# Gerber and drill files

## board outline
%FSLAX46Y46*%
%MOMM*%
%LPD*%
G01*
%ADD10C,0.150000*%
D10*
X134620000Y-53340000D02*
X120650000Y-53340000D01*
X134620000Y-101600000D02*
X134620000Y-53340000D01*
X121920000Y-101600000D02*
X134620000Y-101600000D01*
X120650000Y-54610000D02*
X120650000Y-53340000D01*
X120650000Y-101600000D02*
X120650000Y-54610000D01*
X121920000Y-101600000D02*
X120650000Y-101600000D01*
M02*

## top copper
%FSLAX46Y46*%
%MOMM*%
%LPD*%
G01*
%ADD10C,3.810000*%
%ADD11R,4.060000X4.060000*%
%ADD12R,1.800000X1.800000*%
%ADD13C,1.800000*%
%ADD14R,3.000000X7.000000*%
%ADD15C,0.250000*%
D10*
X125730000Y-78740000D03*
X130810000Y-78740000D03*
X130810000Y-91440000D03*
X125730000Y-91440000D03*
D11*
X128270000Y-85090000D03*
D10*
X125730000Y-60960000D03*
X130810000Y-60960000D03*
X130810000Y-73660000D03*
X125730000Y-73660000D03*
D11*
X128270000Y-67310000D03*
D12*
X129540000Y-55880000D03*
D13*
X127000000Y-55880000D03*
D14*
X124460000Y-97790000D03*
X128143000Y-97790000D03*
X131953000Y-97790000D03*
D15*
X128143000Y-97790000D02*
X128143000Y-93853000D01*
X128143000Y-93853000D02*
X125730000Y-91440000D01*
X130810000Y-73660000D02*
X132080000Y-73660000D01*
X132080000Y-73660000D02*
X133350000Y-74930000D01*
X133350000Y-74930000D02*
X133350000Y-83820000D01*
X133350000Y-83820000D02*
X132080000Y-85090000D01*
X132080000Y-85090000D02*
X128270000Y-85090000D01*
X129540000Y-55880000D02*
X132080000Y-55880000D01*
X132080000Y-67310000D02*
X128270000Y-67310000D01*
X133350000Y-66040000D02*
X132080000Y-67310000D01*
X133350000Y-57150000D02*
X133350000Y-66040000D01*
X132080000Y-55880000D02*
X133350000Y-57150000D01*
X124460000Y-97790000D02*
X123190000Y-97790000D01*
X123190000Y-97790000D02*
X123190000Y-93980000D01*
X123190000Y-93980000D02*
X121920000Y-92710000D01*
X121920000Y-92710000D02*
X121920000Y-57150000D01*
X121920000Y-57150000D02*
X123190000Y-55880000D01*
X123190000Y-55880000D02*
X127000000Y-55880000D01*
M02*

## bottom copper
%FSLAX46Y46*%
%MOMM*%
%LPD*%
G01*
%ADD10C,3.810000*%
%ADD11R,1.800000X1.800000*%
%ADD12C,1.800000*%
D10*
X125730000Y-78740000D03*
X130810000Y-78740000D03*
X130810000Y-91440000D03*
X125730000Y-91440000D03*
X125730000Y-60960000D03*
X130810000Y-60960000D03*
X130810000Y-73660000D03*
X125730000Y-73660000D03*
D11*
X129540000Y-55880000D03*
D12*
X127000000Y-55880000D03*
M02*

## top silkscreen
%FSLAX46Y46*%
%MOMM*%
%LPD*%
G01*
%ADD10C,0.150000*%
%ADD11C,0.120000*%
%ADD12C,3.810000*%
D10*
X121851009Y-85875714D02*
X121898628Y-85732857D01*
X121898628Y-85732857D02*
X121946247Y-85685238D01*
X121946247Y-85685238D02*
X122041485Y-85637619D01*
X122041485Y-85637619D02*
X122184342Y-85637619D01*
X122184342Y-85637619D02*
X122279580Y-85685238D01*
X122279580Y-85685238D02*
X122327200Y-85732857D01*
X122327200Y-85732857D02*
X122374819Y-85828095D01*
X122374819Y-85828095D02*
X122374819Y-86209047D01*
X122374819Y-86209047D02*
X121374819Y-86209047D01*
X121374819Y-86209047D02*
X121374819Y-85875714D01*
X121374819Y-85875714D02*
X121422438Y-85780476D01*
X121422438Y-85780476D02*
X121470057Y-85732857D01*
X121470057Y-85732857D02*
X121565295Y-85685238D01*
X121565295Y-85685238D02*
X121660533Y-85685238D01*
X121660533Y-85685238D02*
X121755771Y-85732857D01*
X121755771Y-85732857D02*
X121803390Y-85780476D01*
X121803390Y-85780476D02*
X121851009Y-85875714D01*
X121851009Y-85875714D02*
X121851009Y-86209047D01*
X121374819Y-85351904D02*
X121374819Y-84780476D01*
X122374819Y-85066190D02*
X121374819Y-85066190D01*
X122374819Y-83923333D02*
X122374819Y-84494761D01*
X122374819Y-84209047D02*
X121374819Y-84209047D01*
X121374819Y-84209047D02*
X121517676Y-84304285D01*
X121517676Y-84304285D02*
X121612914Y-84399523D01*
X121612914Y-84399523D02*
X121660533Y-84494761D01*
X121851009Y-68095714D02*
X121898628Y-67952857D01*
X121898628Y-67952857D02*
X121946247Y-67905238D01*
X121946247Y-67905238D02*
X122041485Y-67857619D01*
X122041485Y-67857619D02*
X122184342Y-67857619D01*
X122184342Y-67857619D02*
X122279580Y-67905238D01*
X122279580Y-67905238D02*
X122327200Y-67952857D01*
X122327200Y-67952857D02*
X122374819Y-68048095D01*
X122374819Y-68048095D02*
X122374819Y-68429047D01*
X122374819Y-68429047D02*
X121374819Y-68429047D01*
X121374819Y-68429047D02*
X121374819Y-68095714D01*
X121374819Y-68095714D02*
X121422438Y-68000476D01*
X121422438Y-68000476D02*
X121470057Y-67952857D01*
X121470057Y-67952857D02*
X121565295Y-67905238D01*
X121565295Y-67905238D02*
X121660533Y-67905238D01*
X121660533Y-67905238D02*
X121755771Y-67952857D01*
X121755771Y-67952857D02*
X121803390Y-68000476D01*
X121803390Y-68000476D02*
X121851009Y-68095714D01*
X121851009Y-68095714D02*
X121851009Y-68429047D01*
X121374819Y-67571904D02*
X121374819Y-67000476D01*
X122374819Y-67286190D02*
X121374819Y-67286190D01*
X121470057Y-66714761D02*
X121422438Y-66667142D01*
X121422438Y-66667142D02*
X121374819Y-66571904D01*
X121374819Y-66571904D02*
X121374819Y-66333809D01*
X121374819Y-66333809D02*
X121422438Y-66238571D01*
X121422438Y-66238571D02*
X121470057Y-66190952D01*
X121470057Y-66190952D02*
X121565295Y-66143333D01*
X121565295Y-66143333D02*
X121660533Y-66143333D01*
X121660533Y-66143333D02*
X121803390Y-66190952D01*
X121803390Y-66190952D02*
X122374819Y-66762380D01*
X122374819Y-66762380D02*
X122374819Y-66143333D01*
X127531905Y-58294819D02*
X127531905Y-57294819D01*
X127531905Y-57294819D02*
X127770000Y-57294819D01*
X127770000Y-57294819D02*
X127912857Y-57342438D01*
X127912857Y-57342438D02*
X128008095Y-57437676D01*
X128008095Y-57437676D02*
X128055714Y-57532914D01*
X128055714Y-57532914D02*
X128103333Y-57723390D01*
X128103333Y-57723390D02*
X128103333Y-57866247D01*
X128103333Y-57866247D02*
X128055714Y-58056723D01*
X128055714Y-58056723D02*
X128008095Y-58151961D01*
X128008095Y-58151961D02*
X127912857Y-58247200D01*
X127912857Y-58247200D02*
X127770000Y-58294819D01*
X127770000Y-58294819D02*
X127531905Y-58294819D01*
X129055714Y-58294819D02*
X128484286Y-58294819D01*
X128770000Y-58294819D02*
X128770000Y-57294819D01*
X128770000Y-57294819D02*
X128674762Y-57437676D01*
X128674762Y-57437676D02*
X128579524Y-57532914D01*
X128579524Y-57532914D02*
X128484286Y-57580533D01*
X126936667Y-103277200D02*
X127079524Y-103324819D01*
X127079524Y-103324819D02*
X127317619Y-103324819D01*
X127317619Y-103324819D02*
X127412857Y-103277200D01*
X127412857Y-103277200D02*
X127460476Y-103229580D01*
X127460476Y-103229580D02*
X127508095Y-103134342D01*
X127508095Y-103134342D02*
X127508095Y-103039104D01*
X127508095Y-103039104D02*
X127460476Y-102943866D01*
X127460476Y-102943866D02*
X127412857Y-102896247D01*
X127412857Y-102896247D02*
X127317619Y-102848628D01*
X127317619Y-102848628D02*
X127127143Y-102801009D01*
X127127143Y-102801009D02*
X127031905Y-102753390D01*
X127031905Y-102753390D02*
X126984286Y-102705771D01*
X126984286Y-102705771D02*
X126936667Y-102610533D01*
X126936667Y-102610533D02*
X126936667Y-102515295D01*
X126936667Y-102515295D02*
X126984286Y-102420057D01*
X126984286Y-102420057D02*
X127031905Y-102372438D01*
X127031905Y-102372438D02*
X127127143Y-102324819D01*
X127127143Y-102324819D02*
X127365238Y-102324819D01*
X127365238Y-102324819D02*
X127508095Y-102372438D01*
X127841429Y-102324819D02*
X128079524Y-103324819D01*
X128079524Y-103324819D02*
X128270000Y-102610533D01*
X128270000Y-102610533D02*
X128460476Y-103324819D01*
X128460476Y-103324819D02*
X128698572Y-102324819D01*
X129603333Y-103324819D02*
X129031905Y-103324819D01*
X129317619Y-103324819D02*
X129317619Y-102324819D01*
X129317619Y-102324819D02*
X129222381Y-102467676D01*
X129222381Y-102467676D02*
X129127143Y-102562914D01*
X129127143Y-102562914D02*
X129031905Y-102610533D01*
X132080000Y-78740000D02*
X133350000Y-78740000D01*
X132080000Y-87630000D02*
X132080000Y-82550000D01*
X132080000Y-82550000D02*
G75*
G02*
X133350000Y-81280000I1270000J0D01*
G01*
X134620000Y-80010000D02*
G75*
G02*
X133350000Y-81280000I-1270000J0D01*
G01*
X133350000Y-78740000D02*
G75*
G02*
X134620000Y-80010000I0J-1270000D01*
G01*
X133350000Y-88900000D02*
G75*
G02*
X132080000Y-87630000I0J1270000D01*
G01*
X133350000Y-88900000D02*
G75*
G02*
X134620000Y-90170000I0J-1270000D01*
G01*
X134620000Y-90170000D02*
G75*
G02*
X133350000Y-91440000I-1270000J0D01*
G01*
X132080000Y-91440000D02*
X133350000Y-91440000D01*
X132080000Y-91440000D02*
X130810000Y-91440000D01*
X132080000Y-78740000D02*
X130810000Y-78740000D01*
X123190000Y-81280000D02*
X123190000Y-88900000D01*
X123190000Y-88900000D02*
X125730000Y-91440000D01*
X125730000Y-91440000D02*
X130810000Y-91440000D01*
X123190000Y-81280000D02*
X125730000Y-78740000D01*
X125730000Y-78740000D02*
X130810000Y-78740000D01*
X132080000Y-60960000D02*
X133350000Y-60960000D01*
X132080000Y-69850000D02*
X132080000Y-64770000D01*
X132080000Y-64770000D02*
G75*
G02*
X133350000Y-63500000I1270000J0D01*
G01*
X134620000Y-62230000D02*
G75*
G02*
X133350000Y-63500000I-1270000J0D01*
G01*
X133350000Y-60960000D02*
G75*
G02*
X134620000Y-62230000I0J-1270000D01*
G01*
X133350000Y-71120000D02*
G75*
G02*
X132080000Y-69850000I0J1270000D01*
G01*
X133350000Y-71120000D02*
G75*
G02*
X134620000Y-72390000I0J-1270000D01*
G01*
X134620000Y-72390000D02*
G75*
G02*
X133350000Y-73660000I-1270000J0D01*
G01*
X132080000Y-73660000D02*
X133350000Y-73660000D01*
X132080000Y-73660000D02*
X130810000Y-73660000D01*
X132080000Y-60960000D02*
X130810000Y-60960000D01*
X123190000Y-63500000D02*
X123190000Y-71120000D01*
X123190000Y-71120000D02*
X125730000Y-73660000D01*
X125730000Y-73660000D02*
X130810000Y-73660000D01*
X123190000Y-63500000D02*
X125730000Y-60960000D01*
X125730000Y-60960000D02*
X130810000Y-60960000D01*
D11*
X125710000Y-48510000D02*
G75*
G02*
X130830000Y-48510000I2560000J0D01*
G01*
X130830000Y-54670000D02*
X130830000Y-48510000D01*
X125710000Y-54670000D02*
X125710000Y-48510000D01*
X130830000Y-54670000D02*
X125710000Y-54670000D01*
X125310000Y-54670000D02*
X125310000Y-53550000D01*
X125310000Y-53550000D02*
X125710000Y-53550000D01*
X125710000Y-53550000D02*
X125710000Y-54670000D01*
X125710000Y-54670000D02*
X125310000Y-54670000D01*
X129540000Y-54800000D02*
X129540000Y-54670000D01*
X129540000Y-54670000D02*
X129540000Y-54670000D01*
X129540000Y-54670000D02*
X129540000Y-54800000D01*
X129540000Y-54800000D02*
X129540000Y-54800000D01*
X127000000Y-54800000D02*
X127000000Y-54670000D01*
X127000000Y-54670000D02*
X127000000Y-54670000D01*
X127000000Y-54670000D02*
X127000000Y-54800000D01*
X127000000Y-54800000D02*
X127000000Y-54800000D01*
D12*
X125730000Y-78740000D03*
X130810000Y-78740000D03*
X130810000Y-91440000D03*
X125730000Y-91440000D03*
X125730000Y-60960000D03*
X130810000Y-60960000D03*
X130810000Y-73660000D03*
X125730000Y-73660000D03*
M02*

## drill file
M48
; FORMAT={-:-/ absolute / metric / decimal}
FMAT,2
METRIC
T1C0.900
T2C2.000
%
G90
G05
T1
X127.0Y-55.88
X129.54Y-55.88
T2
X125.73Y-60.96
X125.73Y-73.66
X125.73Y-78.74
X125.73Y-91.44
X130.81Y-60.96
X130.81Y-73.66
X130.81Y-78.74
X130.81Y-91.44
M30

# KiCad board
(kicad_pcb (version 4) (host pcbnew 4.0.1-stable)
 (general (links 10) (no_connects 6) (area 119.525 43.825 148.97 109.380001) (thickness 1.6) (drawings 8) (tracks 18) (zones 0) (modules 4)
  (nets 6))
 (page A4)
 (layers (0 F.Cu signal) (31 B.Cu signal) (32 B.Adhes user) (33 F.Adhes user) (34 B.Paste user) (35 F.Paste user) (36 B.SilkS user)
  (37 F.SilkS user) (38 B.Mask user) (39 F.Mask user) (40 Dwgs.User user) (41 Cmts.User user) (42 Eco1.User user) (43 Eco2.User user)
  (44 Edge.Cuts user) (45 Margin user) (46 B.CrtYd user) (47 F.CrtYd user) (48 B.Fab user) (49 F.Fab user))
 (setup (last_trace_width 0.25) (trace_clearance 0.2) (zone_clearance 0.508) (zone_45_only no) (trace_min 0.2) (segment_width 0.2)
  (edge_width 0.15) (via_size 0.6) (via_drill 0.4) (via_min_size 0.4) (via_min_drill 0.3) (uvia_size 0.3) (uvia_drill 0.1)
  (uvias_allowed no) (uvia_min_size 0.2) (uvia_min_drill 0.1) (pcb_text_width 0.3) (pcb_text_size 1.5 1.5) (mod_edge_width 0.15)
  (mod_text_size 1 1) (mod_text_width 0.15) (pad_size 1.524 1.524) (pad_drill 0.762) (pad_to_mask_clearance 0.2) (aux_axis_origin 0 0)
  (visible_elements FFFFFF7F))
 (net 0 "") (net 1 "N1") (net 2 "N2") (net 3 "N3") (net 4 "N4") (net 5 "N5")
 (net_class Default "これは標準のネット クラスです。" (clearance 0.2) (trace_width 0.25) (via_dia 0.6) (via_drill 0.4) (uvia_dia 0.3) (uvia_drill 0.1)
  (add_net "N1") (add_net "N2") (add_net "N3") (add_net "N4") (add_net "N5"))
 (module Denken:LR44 (layer F.Cu) (at 128.27 85.09 270)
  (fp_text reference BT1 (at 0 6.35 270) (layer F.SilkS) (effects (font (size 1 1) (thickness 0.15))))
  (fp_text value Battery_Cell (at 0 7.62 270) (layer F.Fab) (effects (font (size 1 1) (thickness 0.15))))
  (fp_line (start -6.35 -3.81) (end -6.35 -5.08) (layer F.SilkS) (width 0.15))
  (fp_line (start 2.54 -3.81) (end -2.54 -3.81) (layer F.SilkS) (width 0.15))
  (fp_arc (start -2.54 -5.08) (end -2.54 -3.81) (angle 90) (layer F.SilkS) (width 0.15))
  (fp_arc (start -5.08 -5.08) (end -5.08 -6.35) (angle 90) (layer F.SilkS) (width 0.15))
  (fp_arc (start -5.08 -5.08) (end -6.35 -5.08) (angle 90) (layer F.SilkS) (width 0.15))
  (fp_arc (start 2.54 -5.08) (end 3.81 -5.08) (angle 90) (layer F.SilkS) (width 0.15))
  (fp_arc (start 5.08 -5.08) (end 3.81 -5.08) (angle 90) (layer F.SilkS) (width 0.15))
  (fp_arc (start 5.08 -5.08) (end 5.08 -6.35) (angle 90) (layer F.SilkS) (width 0.15))
  (fp_line (start 6.35 -3.81) (end 6.35 -5.08) (layer F.SilkS) (width 0.15))
  (fp_line (start 6.35 -3.81) (end 6.35 -2.54) (layer F.SilkS) (width 0.15))
  (fp_line (start -6.35 -3.81) (end -6.35 -2.54) (layer F.SilkS) (width 0.15))
  (fp_line (start -3.81 5.08) (end 3.81 5.08) (layer F.SilkS) (width 0.15))
  (fp_line (start 3.81 5.08) (end 6.35 2.54) (layer F.SilkS) (width 0.15))
  (fp_line (start 6.35 2.54) (end 6.35 -2.54) (layer F.SilkS) (width 0.15))
  (fp_line (start -3.81 5.08) (end -6.35 2.54) (layer F.SilkS) (width 0.15))
  (fp_line (start -6.35 2.54) (end -6.35 -2.54) (layer F.SilkS) (width 0.15))
  (pad 1 thru_hole circle (at -6.35 2.54 270) (size 3.81 3.81) (drill 2) (layers *.Cu *.Mask F.SilkS) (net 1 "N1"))
  (pad 1 thru_hole circle (at -6.35 -2.54 270) (size 3.81 3.81) (drill 2) (layers *.Cu *.Mask F.SilkS) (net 1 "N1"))
  (pad 1 thru_hole circle (at 6.35 -2.54 270) (size 3.81 3.81) (drill 2) (layers *.Cu *.Mask F.SilkS) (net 1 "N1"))
  (pad 1 thru_hole circle (at 6.35 2.54 270) (size 3.81 3.81) (drill 2) (layers *.Cu *.Mask F.SilkS) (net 1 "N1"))
  (pad 2 smd rect (at 0 0 270) (size 4.06 4.06) (layers F.Cu F.Paste F.Mask) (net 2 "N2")))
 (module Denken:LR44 (layer F.Cu) (at 128.27 67.31 270)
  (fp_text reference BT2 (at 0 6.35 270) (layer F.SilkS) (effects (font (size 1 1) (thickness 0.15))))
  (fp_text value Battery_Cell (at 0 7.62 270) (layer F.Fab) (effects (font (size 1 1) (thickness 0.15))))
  (fp_line (start -6.35 -3.81) (end -6.35 -5.08) (layer F.SilkS) (width 0.15))
  (fp_line (start 2.54 -3.81) (end -2.54 -3.81) (layer F.SilkS) (width 0.15))
  (fp_arc (start -2.54 -5.08) (end -2.54 -3.81) (angle 90) (layer F.SilkS) (width 0.15))
  (fp_arc (start -5.08 -5.08) (end -5.08 -6.35) (angle 90) (layer F.SilkS) (width 0.15))
  (fp_arc (start -5.08 -5.08) (end -6.35 -5.08) (angle 90) (layer F.SilkS) (width 0.15))
  (fp_arc (start 2.54 -5.08) (end 3.81 -5.08) (angle 90) (layer F.SilkS) (width 0.15))
  (fp_arc (start 5.08 -5.08) (end 3.81 -5.08) (angle 90) (layer F.SilkS) (width 0.15))
  (fp_arc (start 5.08 -5.08) (end 5.08 -6.35) (angle 90) (layer F.SilkS) (width 0.15))
  (fp_line (start 6.35 -3.81) (end 6.35 -5.08) (layer F.SilkS) (width 0.15))
  (fp_line (start 6.35 -3.81) (end 6.35 -2.54) (layer F.SilkS) (width 0.15))
  (fp_line (start -6.35 -3.81) (end -6.35 -2.54) (layer F.SilkS) (width 0.15))
  (fp_line (start -3.81 5.08) (end 3.81 5.08) (layer F.SilkS) (width 0.15))
  (fp_line (start 3.81 5.08) (end 6.35 2.54) (layer F.SilkS) (width 0.15))
  (fp_line (start 6.35 2.54) (end 6.35 -2.54) (layer F.SilkS) (width 0.15))
  (fp_line (start -3.81 5.08) (end -6.35 2.54) (layer F.SilkS) (width 0.15))
  (fp_line (start -6.35 2.54) (end -6.35 -2.54) (layer F.SilkS) (width 0.15))
  (pad 1 thru_hole circle (at -6.35 2.54 270) (size 3.81 3.81) (drill 2) (layers *.Cu *.Mask F.SilkS) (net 2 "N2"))
  (pad 1 thru_hole circle (at -6.35 -2.54 270) (size 3.81 3.81) (drill 2) (layers *.Cu *.Mask F.SilkS) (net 2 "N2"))
  (pad 1 thru_hole circle (at 6.35 -2.54 270) (size 3.81 3.81) (drill 2) (layers *.Cu *.Mask F.SilkS) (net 2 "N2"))
  (pad 1 thru_hole circle (at 6.35 2.54 270) (size 3.81 3.81) (drill 2) (layers *.Cu *.Mask F.SilkS) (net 2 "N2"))
  (pad 2 smd rect (at 0 0 270) (size 4.06 4.06) (layers F.Cu F.Paste F.Mask) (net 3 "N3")))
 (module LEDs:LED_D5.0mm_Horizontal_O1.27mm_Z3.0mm (layer F.Cu) (at 129.54 55.88 180)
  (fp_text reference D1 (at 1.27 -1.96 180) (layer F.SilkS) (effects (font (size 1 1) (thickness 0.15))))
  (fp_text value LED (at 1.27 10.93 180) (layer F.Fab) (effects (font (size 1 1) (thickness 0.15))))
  (fp_arc (start 1.27 7.37) (end -1.29 7.37) (angle -180) (layer F.SilkS) (width 0.12))
  (fp_line (start -1.29 1.21) (end -1.29 7.37) (layer F.SilkS) (width 0.12))
  (fp_line (start 3.83 1.21) (end 3.83 7.37) (layer F.SilkS) (width 0.12))
  (fp_line (start -1.29 1.21) (end 3.83 1.21) (layer F.SilkS) (width 0.12))
  (fp_line (start 4.23 1.21) (end 4.23 2.33) (layer F.SilkS) (width 0.12))
  (fp_line (start 4.23 2.33) (end 3.83 2.33) (layer F.SilkS) (width 0.12))
  (fp_line (start 3.83 2.33) (end 3.83 1.21) (layer F.SilkS) (width 0.12))
  (fp_line (start 3.83 1.21) (end 4.23 1.21) (layer F.SilkS) (width 0.12))
  (fp_line (start 0 1.08) (end 0 1.21) (layer F.SilkS) (width 0.12))
  (fp_line (start 0 1.21) (end 0 1.21) (layer F.SilkS) (width 0.12))
  (fp_line (start 0 1.21) (end 0 1.08) (layer F.SilkS) (width 0.12))
  (fp_line (start 0 1.08) (end 0 1.08) (layer F.SilkS) (width 0.12))
  (fp_line (start 2.54 1.08) (end 2.54 1.21) (layer F.SilkS) (width 0.12))
  (fp_line (start 2.54 1.21) (end 2.54 1.21) (layer F.SilkS) (width 0.12))
  (fp_line (start 2.54 1.21) (end 2.54 1.08) (layer F.SilkS) (width 0.12))
  (fp_line (start 2.54 1.08) (end 2.54 1.08) (layer F.SilkS) (width 0.12))
  (pad 1 thru_hole rect (at 0 0 180) (size 1.8 1.8) (drill 0.9) (layers *.Cu *.Mask) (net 3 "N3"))
  (pad 2 thru_hole circle (at 2.54 0 180) (size 1.8 1.8) (drill 0.9) (layers *.Cu *.Mask) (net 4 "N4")))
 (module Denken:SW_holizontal (layer F.Cu) (at 128.27 97.79)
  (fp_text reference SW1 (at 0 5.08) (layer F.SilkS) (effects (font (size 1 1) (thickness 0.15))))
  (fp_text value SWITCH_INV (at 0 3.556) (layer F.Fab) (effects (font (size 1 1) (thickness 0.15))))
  (pad 1 smd rect (at -3.81 0) (size 3 7) (layers F.Cu F.Paste F.Mask) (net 4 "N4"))
  (pad 2 smd rect (at -0.127 0) (size 3 7) (layers F.Cu F.Paste F.Mask) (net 1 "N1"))
  (pad 3 smd rect (at 3.683 0) (size 3 7) (layers F.Cu F.Paste F.Mask) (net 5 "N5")))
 (gr_line (start 134.62 53.34) (end 120.65 53.34) (angle 90) (layer Edge.Cuts) (width 0.15))
 (gr_line (start 134.62 101.6) (end 134.62 53.34) (angle 90) (layer Edge.Cuts) (width 0.15))
 (gr_line (start 121.92 101.6) (end 134.62 101.6) (angle 90) (layer Edge.Cuts) (width 0.15))
 (gr_line (start 120.65 54.61) (end 120.65 53.34) (angle 90) (layer Edge.Cuts) (width 0.15))
 (gr_line (start 120.65 101.6) (end 120.65 54.61) (angle 90) (layer Edge.Cuts) (width 0.15))
 (gr_line (start 121.92 101.6) (end 120.65 101.6) (angle 90) (layer Edge.Cuts) (width 0.15))
 (segment (start 128.143 97.79) (end 128.143 93.853) (width 0.25) (layer F.Cu) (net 1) (status 400000))
 (segment (start 128.143 93.853) (end 125.73 91.44) (width 0.25) (layer F.Cu) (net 1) (status 800000))
 (segment (start 130.81 73.66) (end 132.08 73.66) (width 0.25) (layer F.Cu) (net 2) (status C00000))
 (segment (start 132.08 73.66) (end 133.35 74.93) (width 0.25) (layer F.Cu) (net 2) (status 400000))
 (segment (start 133.35 74.93) (end 133.35 83.82) (width 0.25) (layer F.Cu) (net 2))
 (segment (start 133.35 83.82) (end 132.08 85.09) (width 0.25) (layer F.Cu) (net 2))
 (segment (start 132.08 85.09) (end 128.27 85.09) (width 0.25) (layer F.Cu) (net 2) (status 800000))
 (segment (start 129.54 55.88) (end 132.08 55.88) (width 0.25) (layer F.Cu) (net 3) (status 400000))
 (segment (start 132.08 67.31) (end 128.27 67.31) (width 0.25) (layer F.Cu) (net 3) (status 800000))
 (segment (start 133.35 66.04) (end 132.08 67.31) (width 0.25) (layer F.Cu) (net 3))
 (segment (start 133.35 57.15) (end 133.35 66.04) (width 0.25) (layer F.Cu) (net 3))
 (segment (start 132.08 55.88) (end 133.35 57.15) (width 0.25) (layer F.Cu) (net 3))
 (segment (start 124.46 97.79) (end 123.19 97.79) (width 0.25) (layer F.Cu) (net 4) (status C00000))
 (segment (start 123.19 97.79) (end 123.19 93.98) (width 0.25) (layer F.Cu) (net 4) (status 400000))
 (segment (start 123.19 93.98) (end 121.92 92.71) (width 0.25) (layer F.Cu) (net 4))
 (segment (start 121.92 92.71) (end 121.92 57.15) (width 0.25) (layer F.Cu) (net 4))
 (segment (start 121.92 57.15) (end 123.19 55.88) (width 0.25) (layer F.Cu) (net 4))
 (segment (start 123.19 55.88) (end 127 55.88) (width 0.25) (layer F.Cu) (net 4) (status 800000)))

